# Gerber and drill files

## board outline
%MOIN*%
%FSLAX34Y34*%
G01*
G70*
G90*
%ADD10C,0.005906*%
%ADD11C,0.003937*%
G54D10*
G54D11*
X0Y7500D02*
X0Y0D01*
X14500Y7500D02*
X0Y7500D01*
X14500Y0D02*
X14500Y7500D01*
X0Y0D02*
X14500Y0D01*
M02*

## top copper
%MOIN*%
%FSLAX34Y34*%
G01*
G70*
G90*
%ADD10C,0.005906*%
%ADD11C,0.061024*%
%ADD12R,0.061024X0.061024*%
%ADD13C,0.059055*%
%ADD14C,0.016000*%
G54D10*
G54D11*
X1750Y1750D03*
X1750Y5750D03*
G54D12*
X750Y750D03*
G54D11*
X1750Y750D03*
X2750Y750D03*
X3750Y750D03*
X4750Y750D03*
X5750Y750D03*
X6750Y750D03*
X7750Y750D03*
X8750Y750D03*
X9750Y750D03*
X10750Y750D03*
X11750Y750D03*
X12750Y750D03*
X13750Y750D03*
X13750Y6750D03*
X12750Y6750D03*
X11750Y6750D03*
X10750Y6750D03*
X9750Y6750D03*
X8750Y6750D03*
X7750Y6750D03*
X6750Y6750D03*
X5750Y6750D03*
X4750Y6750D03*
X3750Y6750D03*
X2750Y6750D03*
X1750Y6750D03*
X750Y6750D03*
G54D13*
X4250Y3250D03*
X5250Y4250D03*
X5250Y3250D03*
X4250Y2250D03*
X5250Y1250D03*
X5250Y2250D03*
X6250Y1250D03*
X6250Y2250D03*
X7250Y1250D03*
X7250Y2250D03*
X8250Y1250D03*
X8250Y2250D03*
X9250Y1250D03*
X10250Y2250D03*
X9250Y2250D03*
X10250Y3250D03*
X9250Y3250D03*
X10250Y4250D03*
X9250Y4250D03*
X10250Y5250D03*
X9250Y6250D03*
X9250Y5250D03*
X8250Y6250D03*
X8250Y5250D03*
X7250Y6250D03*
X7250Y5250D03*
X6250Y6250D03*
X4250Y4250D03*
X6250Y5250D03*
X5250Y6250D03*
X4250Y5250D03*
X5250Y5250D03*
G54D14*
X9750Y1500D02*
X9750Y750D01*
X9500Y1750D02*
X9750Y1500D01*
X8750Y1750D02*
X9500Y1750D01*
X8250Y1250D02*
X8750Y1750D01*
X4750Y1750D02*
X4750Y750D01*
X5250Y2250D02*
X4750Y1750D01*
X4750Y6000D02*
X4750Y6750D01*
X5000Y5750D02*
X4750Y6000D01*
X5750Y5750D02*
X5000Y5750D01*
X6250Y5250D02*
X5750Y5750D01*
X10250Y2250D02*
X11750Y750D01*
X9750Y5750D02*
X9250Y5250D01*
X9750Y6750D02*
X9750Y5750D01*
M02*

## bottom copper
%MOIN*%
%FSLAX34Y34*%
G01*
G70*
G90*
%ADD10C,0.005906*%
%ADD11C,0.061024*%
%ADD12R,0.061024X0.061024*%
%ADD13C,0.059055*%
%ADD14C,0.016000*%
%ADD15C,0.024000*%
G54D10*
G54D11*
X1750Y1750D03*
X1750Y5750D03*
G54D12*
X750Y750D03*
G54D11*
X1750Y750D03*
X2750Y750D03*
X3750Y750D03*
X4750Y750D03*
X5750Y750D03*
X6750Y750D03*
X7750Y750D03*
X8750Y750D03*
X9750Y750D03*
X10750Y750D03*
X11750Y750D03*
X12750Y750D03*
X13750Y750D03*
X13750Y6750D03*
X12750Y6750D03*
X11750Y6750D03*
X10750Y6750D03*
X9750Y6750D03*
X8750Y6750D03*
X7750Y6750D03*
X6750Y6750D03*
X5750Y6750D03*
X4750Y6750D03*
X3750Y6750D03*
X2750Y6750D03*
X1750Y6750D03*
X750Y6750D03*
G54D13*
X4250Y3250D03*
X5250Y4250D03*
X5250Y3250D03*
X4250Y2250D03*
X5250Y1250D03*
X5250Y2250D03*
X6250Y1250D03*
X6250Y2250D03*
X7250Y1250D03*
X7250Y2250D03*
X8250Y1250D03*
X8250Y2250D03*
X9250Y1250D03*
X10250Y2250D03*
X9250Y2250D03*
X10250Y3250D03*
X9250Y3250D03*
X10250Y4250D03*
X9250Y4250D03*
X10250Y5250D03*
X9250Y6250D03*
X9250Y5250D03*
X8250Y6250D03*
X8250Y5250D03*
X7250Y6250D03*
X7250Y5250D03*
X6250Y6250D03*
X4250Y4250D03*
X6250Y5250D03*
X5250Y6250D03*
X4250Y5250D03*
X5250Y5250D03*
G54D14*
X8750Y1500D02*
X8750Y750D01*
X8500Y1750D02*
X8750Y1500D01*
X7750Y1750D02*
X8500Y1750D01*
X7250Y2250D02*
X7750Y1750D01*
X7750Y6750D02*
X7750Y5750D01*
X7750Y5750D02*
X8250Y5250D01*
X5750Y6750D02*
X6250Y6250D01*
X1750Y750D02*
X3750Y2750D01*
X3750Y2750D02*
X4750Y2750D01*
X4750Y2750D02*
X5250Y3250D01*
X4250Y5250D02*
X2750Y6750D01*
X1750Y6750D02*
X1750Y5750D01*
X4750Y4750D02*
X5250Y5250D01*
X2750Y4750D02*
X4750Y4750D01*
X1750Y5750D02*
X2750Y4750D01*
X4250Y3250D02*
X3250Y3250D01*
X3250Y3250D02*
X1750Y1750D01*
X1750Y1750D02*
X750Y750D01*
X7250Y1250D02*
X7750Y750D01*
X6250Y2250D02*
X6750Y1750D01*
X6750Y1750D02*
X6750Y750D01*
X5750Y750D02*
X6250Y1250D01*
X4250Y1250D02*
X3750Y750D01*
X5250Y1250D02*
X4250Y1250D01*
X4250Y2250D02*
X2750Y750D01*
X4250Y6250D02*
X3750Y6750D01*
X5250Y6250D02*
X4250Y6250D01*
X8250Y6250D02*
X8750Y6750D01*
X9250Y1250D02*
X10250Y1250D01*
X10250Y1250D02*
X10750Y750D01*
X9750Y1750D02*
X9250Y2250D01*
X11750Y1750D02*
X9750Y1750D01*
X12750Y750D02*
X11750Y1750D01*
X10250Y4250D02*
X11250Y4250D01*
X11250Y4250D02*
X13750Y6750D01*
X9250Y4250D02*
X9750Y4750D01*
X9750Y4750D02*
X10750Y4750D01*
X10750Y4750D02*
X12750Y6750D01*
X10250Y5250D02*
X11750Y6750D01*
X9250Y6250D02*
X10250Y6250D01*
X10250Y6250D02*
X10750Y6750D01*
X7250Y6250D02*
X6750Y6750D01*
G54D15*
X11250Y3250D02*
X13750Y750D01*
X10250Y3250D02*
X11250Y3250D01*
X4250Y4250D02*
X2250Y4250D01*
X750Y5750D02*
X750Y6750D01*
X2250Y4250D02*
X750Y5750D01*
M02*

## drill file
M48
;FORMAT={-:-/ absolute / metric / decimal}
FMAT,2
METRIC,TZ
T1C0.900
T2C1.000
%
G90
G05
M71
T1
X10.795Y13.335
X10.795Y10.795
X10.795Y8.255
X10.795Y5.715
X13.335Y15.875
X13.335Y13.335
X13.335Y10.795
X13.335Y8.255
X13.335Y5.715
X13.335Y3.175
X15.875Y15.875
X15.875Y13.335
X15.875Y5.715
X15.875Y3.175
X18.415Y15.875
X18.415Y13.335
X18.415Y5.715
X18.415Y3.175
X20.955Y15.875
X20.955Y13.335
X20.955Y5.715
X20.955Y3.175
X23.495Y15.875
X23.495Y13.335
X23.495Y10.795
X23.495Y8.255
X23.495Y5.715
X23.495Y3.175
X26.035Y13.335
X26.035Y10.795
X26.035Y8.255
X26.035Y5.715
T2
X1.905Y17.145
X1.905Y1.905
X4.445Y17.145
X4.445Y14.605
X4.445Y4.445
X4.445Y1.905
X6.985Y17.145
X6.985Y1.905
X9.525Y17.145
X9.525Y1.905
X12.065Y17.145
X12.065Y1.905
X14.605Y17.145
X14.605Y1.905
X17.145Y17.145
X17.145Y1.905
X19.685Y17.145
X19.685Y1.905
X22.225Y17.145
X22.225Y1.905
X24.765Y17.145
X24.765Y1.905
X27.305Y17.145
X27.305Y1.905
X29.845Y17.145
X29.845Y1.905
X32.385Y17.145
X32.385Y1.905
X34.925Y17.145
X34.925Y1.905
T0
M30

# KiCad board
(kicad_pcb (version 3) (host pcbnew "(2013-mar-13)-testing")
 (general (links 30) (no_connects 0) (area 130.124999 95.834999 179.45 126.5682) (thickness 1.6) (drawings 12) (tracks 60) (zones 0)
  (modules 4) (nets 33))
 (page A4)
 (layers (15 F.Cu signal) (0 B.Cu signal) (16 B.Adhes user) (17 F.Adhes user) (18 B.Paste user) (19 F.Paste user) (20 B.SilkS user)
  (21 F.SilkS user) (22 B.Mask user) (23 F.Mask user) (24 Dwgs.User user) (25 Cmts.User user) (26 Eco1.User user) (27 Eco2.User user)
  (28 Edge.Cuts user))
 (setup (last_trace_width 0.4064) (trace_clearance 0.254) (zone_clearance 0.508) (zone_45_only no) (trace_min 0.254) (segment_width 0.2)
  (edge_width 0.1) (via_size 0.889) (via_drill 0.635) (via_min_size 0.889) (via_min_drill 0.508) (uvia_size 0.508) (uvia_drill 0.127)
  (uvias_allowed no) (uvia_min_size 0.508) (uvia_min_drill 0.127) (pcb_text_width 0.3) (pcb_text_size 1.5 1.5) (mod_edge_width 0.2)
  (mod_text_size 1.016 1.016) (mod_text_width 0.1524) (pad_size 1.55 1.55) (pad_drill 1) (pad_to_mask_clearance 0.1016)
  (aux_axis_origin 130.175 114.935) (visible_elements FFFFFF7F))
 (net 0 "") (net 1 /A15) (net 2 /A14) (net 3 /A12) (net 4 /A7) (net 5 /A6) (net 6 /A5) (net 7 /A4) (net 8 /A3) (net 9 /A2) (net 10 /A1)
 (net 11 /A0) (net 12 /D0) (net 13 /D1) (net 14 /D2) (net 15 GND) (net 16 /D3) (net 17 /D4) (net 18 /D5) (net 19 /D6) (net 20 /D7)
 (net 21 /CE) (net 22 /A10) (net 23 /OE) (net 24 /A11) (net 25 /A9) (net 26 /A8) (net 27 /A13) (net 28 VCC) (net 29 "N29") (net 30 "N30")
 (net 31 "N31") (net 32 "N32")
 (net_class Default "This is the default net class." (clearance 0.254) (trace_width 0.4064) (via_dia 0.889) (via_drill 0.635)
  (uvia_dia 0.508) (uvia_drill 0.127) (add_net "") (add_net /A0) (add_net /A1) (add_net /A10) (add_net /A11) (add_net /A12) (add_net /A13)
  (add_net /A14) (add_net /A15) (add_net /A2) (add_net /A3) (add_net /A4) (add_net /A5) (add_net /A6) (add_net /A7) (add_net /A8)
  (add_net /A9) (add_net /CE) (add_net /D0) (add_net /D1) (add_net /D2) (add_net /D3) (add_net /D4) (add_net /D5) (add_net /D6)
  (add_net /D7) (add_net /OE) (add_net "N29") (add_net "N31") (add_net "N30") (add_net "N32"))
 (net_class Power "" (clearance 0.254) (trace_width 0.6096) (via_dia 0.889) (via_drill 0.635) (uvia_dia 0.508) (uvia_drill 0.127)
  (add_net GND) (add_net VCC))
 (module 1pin (layer F.Cu) (at 134.62 110.49)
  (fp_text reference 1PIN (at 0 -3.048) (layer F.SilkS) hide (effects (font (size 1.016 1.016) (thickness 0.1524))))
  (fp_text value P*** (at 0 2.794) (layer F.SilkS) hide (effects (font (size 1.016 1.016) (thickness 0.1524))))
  (pad 1 thru_hole circle (at 0 0) (size 1.55 1.55) (drill 1) (layers *.Cu *.Mask F.SilkS) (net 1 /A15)))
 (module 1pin (layer F.Cu) (at 134.62 100.33)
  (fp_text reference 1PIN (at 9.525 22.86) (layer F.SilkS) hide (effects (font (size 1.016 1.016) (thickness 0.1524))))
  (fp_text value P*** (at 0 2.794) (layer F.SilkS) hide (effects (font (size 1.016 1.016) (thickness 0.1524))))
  (pad 1 thru_hole circle (at 0 0) (size 1.55 1.55) (drill 1) (layers *.Cu *.Mask F.SilkS) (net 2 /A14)))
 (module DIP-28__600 (layer F.Cu) (at 148.59 105.41)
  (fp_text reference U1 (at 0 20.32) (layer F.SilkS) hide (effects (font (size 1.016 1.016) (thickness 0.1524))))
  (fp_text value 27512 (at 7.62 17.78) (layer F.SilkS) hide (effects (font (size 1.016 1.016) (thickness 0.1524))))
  (pad 1 thru_hole rect (at -16.51 7.62) (size 1.55 1.55) (drill 1) (layers *.Cu *.Mask F.SilkS) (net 1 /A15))
  (pad 2 thru_hole circle (at -13.97 7.62) (size 1.55 1.55) (drill 1) (layers *.Cu *.Mask F.SilkS) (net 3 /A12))
  (pad 3 thru_hole circle (at -11.43 7.62) (size 1.55 1.55) (drill 1) (layers *.Cu *.Mask F.SilkS) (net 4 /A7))
  (pad 4 thru_hole circle (at -8.89 7.62) (size 1.55 1.55) (drill 1) (layers *.Cu *.Mask F.SilkS) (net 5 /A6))
  (pad 5 thru_hole circle (at -6.35 7.62) (size 1.55 1.55) (drill 1) (layers *.Cu *.Mask F.SilkS) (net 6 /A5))
  (pad 6 thru_hole circle (at -3.81 7.62) (size 1.55 1.55) (drill 1) (layers *.Cu *.Mask F.SilkS) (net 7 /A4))
  (pad 7 thru_hole circle (at -1.27 7.62) (size 1.55 1.55) (drill 1) (layers *.Cu *.Mask F.SilkS) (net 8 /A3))
  (pad 8 thru_hole circle (at 1.27 7.62) (size 1.55 1.55) (drill 1) (layers *.Cu *.Mask F.SilkS) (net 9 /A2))
  (pad 9 thru_hole circle (at 3.81 7.62) (size 1.55 1.55) (drill 1) (layers *.Cu *.Mask F.SilkS) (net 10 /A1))
  (pad 10 thru_hole circle (at 6.35 7.62) (size 1.55 1.55) (drill 1) (layers *.Cu *.Mask F.SilkS) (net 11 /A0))
  (pad 11 thru_hole circle (at 8.89 7.62) (size 1.55 1.55) (drill 1) (layers *.Cu *.Mask F.SilkS) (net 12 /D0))
  (pad 12 thru_hole circle (at 11.43 7.62) (size 1.55 1.55) (drill 1) (layers *.Cu *.Mask F.SilkS) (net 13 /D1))
  (pad 13 thru_hole circle (at 13.97 7.62) (size 1.55 1.55) (drill 1) (layers *.Cu *.Mask F.SilkS) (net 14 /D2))
  (pad 14 thru_hole circle (at 16.51 7.62) (size 1.55 1.55) (drill 1) (layers *.Cu *.Mask F.SilkS) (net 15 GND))
  (pad 15 thru_hole circle (at 16.51 -7.62) (size 1.55 1.55) (drill 1) (layers *.Cu *.Mask F.SilkS) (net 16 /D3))
  (pad 16 thru_hole circle (at 13.97 -7.62) (size 1.55 1.55) (drill 1) (layers *.Cu *.Mask F.SilkS) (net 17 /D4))
  (pad 17 thru_hole circle (at 11.43 -7.62) (size 1.55 1.55) (drill 1) (layers *.Cu *.Mask F.SilkS) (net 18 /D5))
  (pad 18 thru_hole circle (at 8.89 -7.62) (size 1.55 1.55) (drill 1) (layers *.Cu *.Mask F.SilkS) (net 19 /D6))
  (pad 19 thru_hole circle (at 6.35 -7.62) (size 1.55 1.55) (drill 1) (layers *.Cu *.Mask F.SilkS) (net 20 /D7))
  (pad 20 thru_hole circle (at 3.81 -7.62) (size 1.55 1.55) (drill 1) (layers *.Cu *.Mask F.SilkS) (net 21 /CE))
  (pad 21 thru_hole circle (at 1.27 -7.62) (size 1.55 1.55) (drill 1) (layers *.Cu *.Mask F.SilkS) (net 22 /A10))
  (pad 22 thru_hole circle (at -1.27 -7.62) (size 1.55 1.55) (drill 1) (layers *.Cu *.Mask F.SilkS) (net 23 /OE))
  (pad 23 thru_hole circle (at -3.81 -7.62) (size 1.55 1.55) (drill 1) (layers *.Cu *.Mask F.SilkS) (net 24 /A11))
  (pad 24 thru_hole circle (at -6.35 -7.62) (size 1.55 1.55) (drill 1) (layers *.Cu *.Mask F.SilkS) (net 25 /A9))
  (pad 25 thru_hole circle (at -8.89 -7.62) (size 1.55 1.55) (drill 1) (layers *.Cu *.Mask F.SilkS) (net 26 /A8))
  (pad 26 thru_hole circle (at -11.43 -7.62) (size 1.55 1.55) (drill 1) (layers *.Cu *.Mask F.SilkS) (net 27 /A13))
  (pad 27 thru_hole circle (at -13.97 -7.62) (size 1.55 1.55) (drill 1) (layers *.Cu *.Mask F.SilkS) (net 2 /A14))
  (pad 28 thru_hole circle (at -16.51 -7.62) (size 1.55 1.55) (drill 1) (layers *.Cu *.Mask F.SilkS) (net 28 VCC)))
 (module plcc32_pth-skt (layer F.Cu) (at 148.59 105.41 270)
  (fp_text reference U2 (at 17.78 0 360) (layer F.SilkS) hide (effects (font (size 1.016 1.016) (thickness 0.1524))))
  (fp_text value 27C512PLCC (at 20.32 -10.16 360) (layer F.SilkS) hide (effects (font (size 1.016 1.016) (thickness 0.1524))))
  (pad 2 thru_hole circle (at 1.27 7.62 270) (size 1.5 1.5) (drill 0.9) (layers *.Cu *.Mask F.SilkS) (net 1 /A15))
  (pad 1 thru_hole circle (at -1.27 5.08 270) (size 1.5 1.5) (drill 0.9) (layers *.Cu *.Mask F.SilkS) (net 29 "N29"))
  (pad 3 thru_hole circle (at 1.27 5.08 270) (size 1.5 1.5) (drill 0.9) (layers *.Cu *.Mask F.SilkS) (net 3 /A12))
  (pad 4 thru_hole circle (at 3.81 7.62 270) (size 1.5 1.5) (drill 0.9) (layers *.Cu *.Mask F.SilkS) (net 4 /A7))
  (pad 5 thru_hole circle (at 6.35 5.08 270) (size 1.5 1.5) (drill 0.9) (layers *.Cu *.Mask F.SilkS) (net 5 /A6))
  (pad 6 thru_hole circle (at 3.81 5.08 270) (size 1.5 1.5) (drill 0.9) (layers *.Cu *.Mask F.SilkS) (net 6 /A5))
  (pad 7 thru_hole circle (at 6.35 2.54 270) (size 1.5 1.5) (drill 0.9) (layers *.Cu *.Mask F.SilkS) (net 7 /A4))
  (pad 8 thru_hole circle (at 3.81 2.54 270) (size 1.5 1.5) (drill 0.9) (layers *.Cu *.Mask F.SilkS) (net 8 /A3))
  (pad 9 thru_hole circle (at 6.35 0 270) (size 1.5 1.5) (drill 0.9) (layers *.Cu *.Mask F.SilkS) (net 9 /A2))
  (pad 10 thru_hole circle (at 3.81 0 270) (size 1.5 1.5) (drill 0.9) (layers *.Cu *.Mask F.SilkS) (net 10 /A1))
  (pad 11 thru_hole circle (at 6.35 -2.54 270) (size 1.5 1.5) (drill 0.9) (layers *.Cu *.Mask F.SilkS) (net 11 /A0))
  (pad 12 thru_hole circle (at 3.81 -2.54 270) (size 1.5 1.5) (drill 0.9) (layers *.Cu *.Mask F.SilkS) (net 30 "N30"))
  (pad 13 thru_hole circle (at 6.35 -5.08 270) (size 1.5 1.5) (drill 0.9) (layers *.Cu *.Mask F.SilkS) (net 12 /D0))
  (pad 14 thru_hole circle (at 3.81 -7.62 270) (size 1.5 1.5) (drill 0.9) (layers *.Cu *.Mask F.SilkS) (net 13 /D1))
  (pad 15 thru_hole circle (at 3.81 -5.08 270) (size 1.5 1.5) (drill 0.9) (layers *.Cu *.Mask F.SilkS) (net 14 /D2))
  (pad 16 thru_hole circle (at 1.27 -7.62 270) (size 1.5 1.5) (drill 0.9) (layers *.Cu *.Mask F.SilkS) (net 15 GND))
  (pad 17 thru_hole circle (at 1.27 -5.08 270) (size 1.5 1.5) (drill 0.9) (layers *.Cu *.Mask F.SilkS) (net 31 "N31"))
  (pad 18 thru_hole circle (at -1.27 -7.62 270) (size 1.5 1.5) (drill 0.9) (layers *.Cu *.Mask F.SilkS) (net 16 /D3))
  (pad 19 thru_hole circle (at -1.27 -5.08 270) (size 1.5 1.5) (drill 0.9) (layers *.Cu *.Mask F.SilkS) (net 17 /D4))
  (pad 20 thru_hole circle (at -3.81 -7.62 270) (size 1.5 1.5) (drill 0.9) (layers *.Cu *.Mask F.SilkS) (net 18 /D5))
  (pad 21 thru_hole circle (at -6.35 -5.08 270) (size 1.5 1.5) (drill 0.9) (layers *.Cu *.Mask F.SilkS) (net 19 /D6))
  (pad 22 thru_hole circle (at -3.81 -5.08 270) (size 1.5 1.5) (drill 0.9) (layers *.Cu *.Mask F.SilkS) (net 20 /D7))
  (pad 23 thru_hole circle (at -6.35 -2.54 270) (size 1.5 1.5) (drill 0.9) (layers *.Cu *.Mask F.SilkS) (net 21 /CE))
  (pad 24 thru_hole circle (at -3.81 -2.54 270) (size 1.5 1.5) (drill 0.9) (layers *.Cu *.Mask F.SilkS) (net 22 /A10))
  (pad 25 thru_hole circle (at -6.35 0 270) (size 1.5 1.5) (drill 0.9) (layers *.Cu *.Mask F.SilkS) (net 23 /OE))
  (pad 26 thru_hole circle (at -3.81 0 270) (size 1.5 1.5) (drill 0.9) (layers *.Cu *.Mask F.SilkS) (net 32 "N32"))
  (pad 27 thru_hole circle (at -6.35 2.54 270) (size 1.5 1.5) (drill 0.9) (layers *.Cu *.Mask F.SilkS) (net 24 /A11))
  (pad 32 thru_hole circle (at -1.27 7.62 270) (size 1.5 1.5) (drill 0.9) (layers *.Cu *.Mask F.SilkS) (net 28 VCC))
  (pad 28 thru_hole circle (at -3.81 2.54 270) (size 1.5 1.5) (drill 0.9) (layers *.Cu *.Mask F.SilkS) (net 25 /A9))
  (pad 29 thru_hole circle (at -6.35 5.08 270) (size 1.5 1.5) (drill 0.9) (layers *.Cu *.Mask F.SilkS) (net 26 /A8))
  (pad 30 thru_hole circle (at -3.81 7.62 270) (size 1.5 1.5) (drill 0.9) (layers *.Cu *.Mask F.SilkS) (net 27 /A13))
  (pad 31 thru_hole circle (at -3.81 5.08 270) (size 1.5 1.5) (drill 0.9) (layers *.Cu *.Mask F.SilkS) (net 2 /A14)))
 (gr_line (start 130.175 95.885) (end 130.175 114.935) (angle 90) (layer Edge.Cuts) (width 0.1))
 (gr_line (start 167.005 95.885) (end 130.175 95.885) (angle 90) (layer Edge.Cuts) (width 0.1))
 (gr_line (start 167.005 114.935) (end 167.005 95.885) (angle 90) (layer Edge.Cuts) (width 0.1))
 (gr_line (start 130.175 114.935) (end 167.005 114.935) (angle 90) (layer Edge.Cuts) (width 0.1))
 (segment (start 154.94 111.125) (end 154.94 113.03) (width 0.4064) (layer F.Cu) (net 11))
 (segment (start 154.305 110.49) (end 154.94 111.125) (width 0.4064) (layer F.Cu) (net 11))
 (segment (start 152.4 110.49) (end 154.305 110.49) (width 0.4064) (layer F.Cu) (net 11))
 (segment (start 151.13 111.76) (end 152.4 110.49) (width 0.4064) (layer F.Cu) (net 11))
 (segment (start 152.4 111.125) (end 152.4 113.03) (width 0.4064) (layer B.Cu) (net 10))
 (segment (start 151.765 110.49) (end 152.4 111.125) (width 0.4064) (layer B.Cu) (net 10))
 (segment (start 149.86 110.49) (end 151.765 110.49) (width 0.4064) (layer B.Cu) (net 10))
 (segment (start 148.59 109.22) (end 149.86 110.49) (width 0.4064) (layer B.Cu) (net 10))
 (segment (start 149.86 97.79) (end 149.86 100.33) (width 0.4064) (layer B.Cu) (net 22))
 (segment (start 149.86 100.33) (end 151.13 101.6) (width 0.4064) (layer B.Cu) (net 22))
 (segment (start 144.78 97.79) (end 146.05 99.06) (width 0.4064) (layer B.Cu) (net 24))
 (segment (start 134.62 113.03) (end 139.7 107.95) (width 0.4064) (layer B.Cu) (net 3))
 (segment (start 139.7 107.95) (end 142.24 107.95) (width 0.4064) (layer B.Cu) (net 3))
 (segment (start 142.24 107.95) (end 143.51 106.68) (width 0.4064) (layer B.Cu) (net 3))
 (segment (start 140.97 101.6) (end 137.16 97.79) (width 0.4064) (layer B.Cu) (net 27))
 (segment (start 134.62 97.79) (end 134.62 100.33) (width 0.4064) (layer B.Cu) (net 2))
 (segment (start 142.24 102.87) (end 143.51 101.6) (width 0.4064) (layer B.Cu) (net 2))
 (segment (start 137.16 102.87) (end 142.24 102.87) (width 0.4064) (layer B.Cu) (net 2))
 (segment (start 134.62 100.33) (end 137.16 102.87) (width 0.4064) (layer B.Cu) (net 2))
 (segment (start 140.97 106.68) (end 138.43 106.68) (width 0.4064) (layer B.Cu) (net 1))
 (segment (start 138.43 106.68) (end 134.62 110.49) (width 0.4064) (layer B.Cu) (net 1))
 (segment (start 134.62 110.49) (end 132.08 113.03) (width 0.4064) (layer B.Cu) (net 1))
 (segment (start 148.59 111.76) (end 149.86 113.03) (width 0.4064) (layer B.Cu) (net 9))
 (segment (start 146.05 109.22) (end 147.32 110.49) (width 0.4064) (layer B.Cu) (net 8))
 (segment (start 147.32 110.49) (end 147.32 113.03) (width 0.4064) (layer B.Cu) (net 8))
 (segment (start 144.78 113.03) (end 146.05 111.76) (width 0.4064) (layer B.Cu) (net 7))
 (segment (start 142.24 110.49) (end 142.24 113.03) (width 0.4064) (layer F.Cu) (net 6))
 (segment (start 143.51 109.22) (end 142.24 110.49) (width 0.4064) (layer F.Cu) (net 6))
 (segment (start 140.97 111.76) (end 139.7 113.03) (width 0.4064) (layer B.Cu) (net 5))
 (segment (start 143.51 111.76) (end 140.97 111.76) (width 0.4064) (layer B.Cu) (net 5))
 (segment (start 140.97 109.22) (end 137.16 113.03) (width 0.4064) (layer B.Cu) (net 4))
 (segment (start 140.97 99.06) (end 139.7 97.79) (width 0.4064) (layer B.Cu) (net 26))
 (segment (start 143.51 99.06) (end 140.97 99.06) (width 0.4064) (layer B.Cu) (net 26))
 (segment (start 142.24 99.695) (end 142.24 97.79) (width 0.4064) (layer F.Cu) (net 25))
 (segment (start 142.875 100.33) (end 142.24 99.695) (width 0.4064) (layer F.Cu) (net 25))
 (segment (start 144.78 100.33) (end 142.875 100.33) (width 0.4064) (layer F.Cu) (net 25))
 (segment (start 146.05 101.6) (end 144.78 100.33) (width 0.4064) (layer F.Cu) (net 25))
 (segment (start 151.13 99.06) (end 152.4 97.79) (width 0.4064) (layer B.Cu) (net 21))
 (segment (start 153.67 111.76) (end 156.21 111.76) (width 0.4064) (layer B.Cu) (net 12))
 (segment (start 156.21 111.76) (end 157.48 113.03) (width 0.4064) (layer B.Cu) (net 12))
 (segment (start 156.21 109.22) (end 160.02 113.03) (width 0.4064) (layer F.Cu) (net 13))
 (segment (start 154.94 110.49) (end 153.67 109.22) (width 0.4064) (layer B.Cu) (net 14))
 (segment (start 160.02 110.49) (end 154.94 110.49) (width 0.4064) (layer B.Cu) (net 14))
 (segment (start 162.56 113.03) (end 160.02 110.49) (width 0.4064) (layer B.Cu) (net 14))
 (segment (start 156.21 104.14) (end 158.75 104.14) (width 0.4064) (layer B.Cu) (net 16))
 (segment (start 158.75 104.14) (end 165.1 97.79) (width 0.4064) (layer B.Cu) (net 16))
 (segment (start 153.67 104.14) (end 154.94 102.87) (width 0.4064) (layer B.Cu) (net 17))
 (segment (start 154.94 102.87) (end 157.48 102.87) (width 0.4064) (layer B.Cu) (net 17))
 (segment (start 157.48 102.87) (end 162.56 97.79) (width 0.4064) (layer B.Cu) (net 17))
 (segment (start 156.21 101.6) (end 160.02 97.79) (width 0.4064) (layer B.Cu) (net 18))
 (segment (start 153.67 99.06) (end 156.21 99.06) (width 0.4064) (layer B.Cu) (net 19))
 (segment (start 156.21 99.06) (end 157.48 97.79) (width 0.4064) (layer B.Cu) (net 19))
 (segment (start 154.94 100.33) (end 153.67 101.6) (width 0.4064) (layer F.Cu) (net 20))
 (segment (start 154.94 97.79) (end 154.94 100.33) (width 0.4064) (layer F.Cu) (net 20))
 (segment (start 148.59 99.06) (end 147.32 97.79) (width 0.4064) (layer B.Cu) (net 23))
 (segment (start 158.75 106.68) (end 165.1 113.03) (width 0.6096) (layer B.Cu) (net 15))
 (segment (start 156.21 106.68) (end 158.75 106.68) (width 0.6096) (layer B.Cu) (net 15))
 (segment (start 140.97 104.14) (end 135.89 104.14) (width 0.6096) (layer B.Cu) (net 28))
 (segment (start 132.08 100.33) (end 132.08 97.79) (width 0.6096) (layer B.Cu) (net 28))
 (segment (start 135.89 104.14) (end 132.08 100.33) (width 0.6096) (layer B.Cu) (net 28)))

